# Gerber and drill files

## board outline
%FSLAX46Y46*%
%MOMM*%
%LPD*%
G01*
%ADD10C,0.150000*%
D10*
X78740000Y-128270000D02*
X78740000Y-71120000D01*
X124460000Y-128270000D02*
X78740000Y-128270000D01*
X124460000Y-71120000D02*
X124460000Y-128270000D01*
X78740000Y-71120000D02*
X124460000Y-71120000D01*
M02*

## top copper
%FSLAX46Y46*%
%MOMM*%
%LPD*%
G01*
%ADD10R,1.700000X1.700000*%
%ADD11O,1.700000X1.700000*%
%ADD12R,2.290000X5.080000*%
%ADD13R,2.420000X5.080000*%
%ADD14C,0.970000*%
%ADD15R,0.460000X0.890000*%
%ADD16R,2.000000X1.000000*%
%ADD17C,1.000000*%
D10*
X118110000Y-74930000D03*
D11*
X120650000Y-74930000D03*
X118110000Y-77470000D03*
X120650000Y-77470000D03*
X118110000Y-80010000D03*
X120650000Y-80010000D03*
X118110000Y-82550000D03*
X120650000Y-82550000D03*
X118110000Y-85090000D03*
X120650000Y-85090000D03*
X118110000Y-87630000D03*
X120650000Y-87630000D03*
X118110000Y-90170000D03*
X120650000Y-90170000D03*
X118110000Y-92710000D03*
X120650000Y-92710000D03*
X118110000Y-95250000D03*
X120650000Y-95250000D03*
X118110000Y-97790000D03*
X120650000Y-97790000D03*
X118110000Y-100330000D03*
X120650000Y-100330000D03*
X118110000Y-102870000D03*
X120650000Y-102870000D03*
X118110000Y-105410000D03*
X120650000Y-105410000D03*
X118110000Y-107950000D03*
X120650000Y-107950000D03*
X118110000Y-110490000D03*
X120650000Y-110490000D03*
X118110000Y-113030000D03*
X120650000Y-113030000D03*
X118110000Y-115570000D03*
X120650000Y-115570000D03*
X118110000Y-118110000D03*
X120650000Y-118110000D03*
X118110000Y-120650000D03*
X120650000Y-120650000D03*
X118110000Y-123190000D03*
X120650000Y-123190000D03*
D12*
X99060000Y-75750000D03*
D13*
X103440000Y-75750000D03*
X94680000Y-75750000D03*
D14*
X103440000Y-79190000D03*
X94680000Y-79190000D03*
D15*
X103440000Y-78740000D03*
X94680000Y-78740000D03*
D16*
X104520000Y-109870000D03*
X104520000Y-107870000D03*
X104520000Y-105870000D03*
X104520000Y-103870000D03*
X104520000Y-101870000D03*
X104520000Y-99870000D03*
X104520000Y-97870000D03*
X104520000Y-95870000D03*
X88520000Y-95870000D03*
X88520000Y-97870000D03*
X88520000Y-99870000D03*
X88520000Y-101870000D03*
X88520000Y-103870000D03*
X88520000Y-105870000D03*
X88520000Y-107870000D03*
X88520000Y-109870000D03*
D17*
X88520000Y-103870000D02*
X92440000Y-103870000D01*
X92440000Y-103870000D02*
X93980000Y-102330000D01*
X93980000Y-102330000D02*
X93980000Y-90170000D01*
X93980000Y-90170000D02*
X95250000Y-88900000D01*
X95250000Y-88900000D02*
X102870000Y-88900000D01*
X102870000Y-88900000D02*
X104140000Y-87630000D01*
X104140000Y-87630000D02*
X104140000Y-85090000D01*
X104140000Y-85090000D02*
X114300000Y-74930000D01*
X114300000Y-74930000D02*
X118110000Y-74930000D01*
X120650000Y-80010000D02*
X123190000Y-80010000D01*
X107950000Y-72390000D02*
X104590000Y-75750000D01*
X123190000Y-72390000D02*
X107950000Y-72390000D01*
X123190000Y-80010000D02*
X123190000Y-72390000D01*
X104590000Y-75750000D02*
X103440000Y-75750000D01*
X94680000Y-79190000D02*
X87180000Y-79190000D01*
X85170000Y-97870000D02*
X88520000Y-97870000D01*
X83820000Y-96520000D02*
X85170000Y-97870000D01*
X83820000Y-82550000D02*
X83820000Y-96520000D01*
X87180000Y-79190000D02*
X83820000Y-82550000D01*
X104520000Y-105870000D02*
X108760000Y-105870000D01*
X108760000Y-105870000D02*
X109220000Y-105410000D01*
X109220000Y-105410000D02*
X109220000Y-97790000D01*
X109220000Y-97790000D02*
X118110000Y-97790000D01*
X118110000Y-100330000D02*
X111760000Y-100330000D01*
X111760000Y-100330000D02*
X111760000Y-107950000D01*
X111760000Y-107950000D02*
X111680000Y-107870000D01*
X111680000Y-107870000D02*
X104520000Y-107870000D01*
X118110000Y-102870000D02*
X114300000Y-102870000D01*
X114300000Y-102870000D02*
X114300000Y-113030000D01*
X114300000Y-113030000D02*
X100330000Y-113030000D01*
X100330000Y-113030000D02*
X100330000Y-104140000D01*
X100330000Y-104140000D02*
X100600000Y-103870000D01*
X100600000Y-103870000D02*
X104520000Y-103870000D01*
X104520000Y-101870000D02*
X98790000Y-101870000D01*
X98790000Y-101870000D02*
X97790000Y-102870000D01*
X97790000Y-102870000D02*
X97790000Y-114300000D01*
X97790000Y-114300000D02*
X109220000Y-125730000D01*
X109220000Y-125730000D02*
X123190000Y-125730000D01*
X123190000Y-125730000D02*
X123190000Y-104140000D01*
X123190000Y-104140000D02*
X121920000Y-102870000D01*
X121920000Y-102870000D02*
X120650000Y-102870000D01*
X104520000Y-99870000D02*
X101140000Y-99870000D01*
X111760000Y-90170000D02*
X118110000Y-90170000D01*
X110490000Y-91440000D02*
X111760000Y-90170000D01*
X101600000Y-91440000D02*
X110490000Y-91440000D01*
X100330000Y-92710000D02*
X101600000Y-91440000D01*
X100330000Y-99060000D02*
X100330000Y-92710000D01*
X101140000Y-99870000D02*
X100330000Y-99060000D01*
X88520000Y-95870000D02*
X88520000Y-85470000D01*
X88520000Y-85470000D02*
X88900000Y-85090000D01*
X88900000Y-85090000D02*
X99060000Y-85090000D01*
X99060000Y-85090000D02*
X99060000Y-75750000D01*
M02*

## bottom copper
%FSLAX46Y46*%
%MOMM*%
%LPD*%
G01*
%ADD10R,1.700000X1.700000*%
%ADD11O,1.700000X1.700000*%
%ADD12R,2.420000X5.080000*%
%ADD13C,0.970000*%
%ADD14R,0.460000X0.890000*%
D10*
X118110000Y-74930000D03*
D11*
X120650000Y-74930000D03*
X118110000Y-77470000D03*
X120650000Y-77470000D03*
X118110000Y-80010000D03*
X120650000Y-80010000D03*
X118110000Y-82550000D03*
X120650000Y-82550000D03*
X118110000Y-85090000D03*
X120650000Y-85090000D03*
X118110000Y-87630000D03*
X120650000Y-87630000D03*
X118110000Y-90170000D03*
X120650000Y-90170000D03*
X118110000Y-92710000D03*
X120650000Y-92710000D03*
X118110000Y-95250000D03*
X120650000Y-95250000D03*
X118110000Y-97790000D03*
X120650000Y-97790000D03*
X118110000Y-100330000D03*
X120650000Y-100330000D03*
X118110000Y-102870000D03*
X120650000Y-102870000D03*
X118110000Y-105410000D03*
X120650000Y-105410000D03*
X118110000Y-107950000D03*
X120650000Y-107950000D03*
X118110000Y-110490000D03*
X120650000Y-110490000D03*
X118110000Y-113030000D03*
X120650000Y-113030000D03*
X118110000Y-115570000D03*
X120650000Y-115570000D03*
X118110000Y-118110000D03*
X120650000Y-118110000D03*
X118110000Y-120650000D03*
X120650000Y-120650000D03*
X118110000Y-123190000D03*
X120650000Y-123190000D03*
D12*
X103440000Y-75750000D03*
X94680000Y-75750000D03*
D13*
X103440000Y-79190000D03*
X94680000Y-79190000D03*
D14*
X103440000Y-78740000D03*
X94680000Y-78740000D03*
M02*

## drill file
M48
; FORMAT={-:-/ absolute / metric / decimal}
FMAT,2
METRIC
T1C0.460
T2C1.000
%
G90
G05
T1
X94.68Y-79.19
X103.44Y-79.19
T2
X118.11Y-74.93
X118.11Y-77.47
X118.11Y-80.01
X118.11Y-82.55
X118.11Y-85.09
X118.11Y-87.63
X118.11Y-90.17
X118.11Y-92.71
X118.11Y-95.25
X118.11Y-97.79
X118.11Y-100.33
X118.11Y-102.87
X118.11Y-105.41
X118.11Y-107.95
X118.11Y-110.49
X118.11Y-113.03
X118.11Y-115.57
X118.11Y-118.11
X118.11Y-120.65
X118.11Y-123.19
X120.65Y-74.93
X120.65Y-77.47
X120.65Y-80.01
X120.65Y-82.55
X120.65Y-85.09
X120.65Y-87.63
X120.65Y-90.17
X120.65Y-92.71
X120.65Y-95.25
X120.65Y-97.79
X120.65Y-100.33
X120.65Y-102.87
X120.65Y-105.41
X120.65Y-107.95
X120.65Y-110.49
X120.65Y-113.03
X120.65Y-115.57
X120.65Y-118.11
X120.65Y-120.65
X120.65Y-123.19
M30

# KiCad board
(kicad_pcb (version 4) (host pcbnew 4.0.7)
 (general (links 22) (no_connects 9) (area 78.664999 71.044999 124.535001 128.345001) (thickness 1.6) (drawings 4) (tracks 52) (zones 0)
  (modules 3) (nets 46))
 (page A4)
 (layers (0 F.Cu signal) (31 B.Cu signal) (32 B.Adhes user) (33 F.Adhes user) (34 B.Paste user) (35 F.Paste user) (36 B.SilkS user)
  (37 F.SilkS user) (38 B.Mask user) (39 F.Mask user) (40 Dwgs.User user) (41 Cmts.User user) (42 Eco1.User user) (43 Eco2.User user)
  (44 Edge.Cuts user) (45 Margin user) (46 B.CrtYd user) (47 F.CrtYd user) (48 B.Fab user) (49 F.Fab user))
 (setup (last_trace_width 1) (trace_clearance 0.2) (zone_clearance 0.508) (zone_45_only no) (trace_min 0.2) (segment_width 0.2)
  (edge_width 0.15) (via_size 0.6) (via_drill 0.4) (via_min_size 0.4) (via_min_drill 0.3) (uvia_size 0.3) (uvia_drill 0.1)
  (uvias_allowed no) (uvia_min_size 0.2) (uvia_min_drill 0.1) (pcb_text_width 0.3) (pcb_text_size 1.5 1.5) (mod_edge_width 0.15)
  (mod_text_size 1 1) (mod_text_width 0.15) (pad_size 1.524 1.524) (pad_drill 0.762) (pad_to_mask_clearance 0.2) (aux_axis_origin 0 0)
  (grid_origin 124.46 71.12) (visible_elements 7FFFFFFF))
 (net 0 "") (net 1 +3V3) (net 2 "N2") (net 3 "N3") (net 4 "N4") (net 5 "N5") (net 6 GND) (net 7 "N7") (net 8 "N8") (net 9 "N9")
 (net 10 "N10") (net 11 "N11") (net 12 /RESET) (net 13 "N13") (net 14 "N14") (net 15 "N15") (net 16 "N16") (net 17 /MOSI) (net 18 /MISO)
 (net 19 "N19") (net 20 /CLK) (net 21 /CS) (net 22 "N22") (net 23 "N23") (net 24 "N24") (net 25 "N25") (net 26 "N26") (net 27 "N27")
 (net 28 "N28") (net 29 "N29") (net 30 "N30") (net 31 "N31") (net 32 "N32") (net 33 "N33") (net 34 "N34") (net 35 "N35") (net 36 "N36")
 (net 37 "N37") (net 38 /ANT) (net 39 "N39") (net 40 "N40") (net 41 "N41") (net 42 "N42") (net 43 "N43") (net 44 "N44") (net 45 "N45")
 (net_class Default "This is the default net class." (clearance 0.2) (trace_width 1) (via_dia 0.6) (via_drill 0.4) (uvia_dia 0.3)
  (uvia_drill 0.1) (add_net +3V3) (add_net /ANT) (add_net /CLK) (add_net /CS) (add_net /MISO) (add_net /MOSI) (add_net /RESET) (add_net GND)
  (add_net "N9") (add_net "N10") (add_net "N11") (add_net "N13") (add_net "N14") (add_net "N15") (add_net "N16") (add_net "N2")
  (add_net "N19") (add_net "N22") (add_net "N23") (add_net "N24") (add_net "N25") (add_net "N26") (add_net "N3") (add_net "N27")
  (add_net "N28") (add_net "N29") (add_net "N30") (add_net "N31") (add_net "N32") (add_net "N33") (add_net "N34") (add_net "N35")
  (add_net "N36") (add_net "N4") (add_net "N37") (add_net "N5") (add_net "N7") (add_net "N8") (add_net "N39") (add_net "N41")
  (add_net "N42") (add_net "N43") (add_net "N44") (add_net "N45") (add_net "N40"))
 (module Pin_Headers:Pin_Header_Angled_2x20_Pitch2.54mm (layer F.Cu) (at 118.11 74.93)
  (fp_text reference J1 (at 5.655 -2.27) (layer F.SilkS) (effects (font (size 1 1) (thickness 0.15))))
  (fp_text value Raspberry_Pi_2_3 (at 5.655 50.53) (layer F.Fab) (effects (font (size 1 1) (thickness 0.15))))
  (pad 1 thru_hole rect (at 0 0) (size 1.7 1.7) (drill 1) (layers *.Cu *.Mask) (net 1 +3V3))
  (pad 2 thru_hole oval (at 2.54 0) (size 1.7 1.7) (drill 1) (layers *.Cu *.Mask) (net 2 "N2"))
  (pad 3 thru_hole oval (at 0 2.54) (size 1.7 1.7) (drill 1) (layers *.Cu *.Mask) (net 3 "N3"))
  (pad 4 thru_hole oval (at 2.54 2.54) (size 1.7 1.7) (drill 1) (layers *.Cu *.Mask) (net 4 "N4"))
  (pad 5 thru_hole oval (at 0 5.08) (size 1.7 1.7) (drill 1) (layers *.Cu *.Mask) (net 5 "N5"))
  (pad 6 thru_hole oval (at 2.54 5.08) (size 1.7 1.7) (drill 1) (layers *.Cu *.Mask) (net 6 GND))
  (pad 7 thru_hole oval (at 0 7.62) (size 1.7 1.7) (drill 1) (layers *.Cu *.Mask) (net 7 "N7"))
  (pad 8 thru_hole oval (at 2.54 7.62) (size 1.7 1.7) (drill 1) (layers *.Cu *.Mask) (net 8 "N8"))
  (pad 9 thru_hole oval (at 0 10.16) (size 1.7 1.7) (drill 1) (layers *.Cu *.Mask) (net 6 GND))
  (pad 10 thru_hole oval (at 2.54 10.16) (size 1.7 1.7) (drill 1) (layers *.Cu *.Mask) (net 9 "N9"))
  (pad 11 thru_hole oval (at 0 12.7) (size 1.7 1.7) (drill 1) (layers *.Cu *.Mask) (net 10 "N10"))
  (pad 12 thru_hole oval (at 2.54 12.7) (size 1.7 1.7) (drill 1) (layers *.Cu *.Mask) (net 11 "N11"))
  (pad 13 thru_hole oval (at 0 15.24) (size 1.7 1.7) (drill 1) (layers *.Cu *.Mask) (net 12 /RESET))
  (pad 14 thru_hole oval (at 2.54 15.24) (size 1.7 1.7) (drill 1) (layers *.Cu *.Mask) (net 6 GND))
  (pad 15 thru_hole oval (at 0 17.78) (size 1.7 1.7) (drill 1) (layers *.Cu *.Mask) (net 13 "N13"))
  (pad 16 thru_hole oval (at 2.54 17.78) (size 1.7 1.7) (drill 1) (layers *.Cu *.Mask) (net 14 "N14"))
  (pad 17 thru_hole oval (at 0 20.32) (size 1.7 1.7) (drill 1) (layers *.Cu *.Mask) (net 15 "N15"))
  (pad 18 thru_hole oval (at 2.54 20.32) (size 1.7 1.7) (drill 1) (layers *.Cu *.Mask) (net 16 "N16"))
  (pad 19 thru_hole oval (at 0 22.86) (size 1.7 1.7) (drill 1) (layers *.Cu *.Mask) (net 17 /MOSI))
  (pad 20 thru_hole oval (at 2.54 22.86) (size 1.7 1.7) (drill 1) (layers *.Cu *.Mask) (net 6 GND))
  (pad 21 thru_hole oval (at 0 25.4) (size 1.7 1.7) (drill 1) (layers *.Cu *.Mask) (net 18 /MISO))
  (pad 22 thru_hole oval (at 2.54 25.4) (size 1.7 1.7) (drill 1) (layers *.Cu *.Mask) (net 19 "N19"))
  (pad 23 thru_hole oval (at 0 27.94) (size 1.7 1.7) (drill 1) (layers *.Cu *.Mask) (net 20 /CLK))
  (pad 24 thru_hole oval (at 2.54 27.94) (size 1.7 1.7) (drill 1) (layers *.Cu *.Mask) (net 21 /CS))
  (pad 25 thru_hole oval (at 0 30.48) (size 1.7 1.7) (drill 1) (layers *.Cu *.Mask) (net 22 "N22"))
  (pad 26 thru_hole oval (at 2.54 30.48) (size 1.7 1.7) (drill 1) (layers *.Cu *.Mask) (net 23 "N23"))
  (pad 27 thru_hole oval (at 0 33.02) (size 1.7 1.7) (drill 1) (layers *.Cu *.Mask) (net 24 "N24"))
  (pad 28 thru_hole oval (at 2.54 33.02) (size 1.7 1.7) (drill 1) (layers *.Cu *.Mask) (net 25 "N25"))
  (pad 29 thru_hole oval (at 0 35.56) (size 1.7 1.7) (drill 1) (layers *.Cu *.Mask) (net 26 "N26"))
  (pad 30 thru_hole oval (at 2.54 35.56) (size 1.7 1.7) (drill 1) (layers *.Cu *.Mask) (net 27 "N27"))
  (pad 31 thru_hole oval (at 0 38.1) (size 1.7 1.7) (drill 1) (layers *.Cu *.Mask) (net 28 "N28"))
  (pad 32 thru_hole oval (at 2.54 38.1) (size 1.7 1.7) (drill 1) (layers *.Cu *.Mask) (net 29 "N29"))
  (pad 33 thru_hole oval (at 0 40.64) (size 1.7 1.7) (drill 1) (layers *.Cu *.Mask) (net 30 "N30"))
  (pad 34 thru_hole oval (at 2.54 40.64) (size 1.7 1.7) (drill 1) (layers *.Cu *.Mask) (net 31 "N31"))
  (pad 35 thru_hole oval (at 0 43.18) (size 1.7 1.7) (drill 1) (layers *.Cu *.Mask) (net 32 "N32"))
  (pad 36 thru_hole oval (at 2.54 43.18) (size 1.7 1.7) (drill 1) (layers *.Cu *.Mask) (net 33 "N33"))
  (pad 37 thru_hole oval (at 0 45.72) (size 1.7 1.7) (drill 1) (layers *.Cu *.Mask) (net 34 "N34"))
  (pad 38 thru_hole oval (at 2.54 45.72) (size 1.7 1.7) (drill 1) (layers *.Cu *.Mask) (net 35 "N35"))
  (pad 39 thru_hole oval (at 0 48.26) (size 1.7 1.7) (drill 1) (layers *.Cu *.Mask) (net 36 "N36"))
  (pad 40 thru_hole oval (at 2.54 48.26) (size 1.7 1.7) (drill 1) (layers *.Cu *.Mask) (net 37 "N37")))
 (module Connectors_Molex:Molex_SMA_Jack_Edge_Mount (layer F.Cu) (at 99.06 77.47 270)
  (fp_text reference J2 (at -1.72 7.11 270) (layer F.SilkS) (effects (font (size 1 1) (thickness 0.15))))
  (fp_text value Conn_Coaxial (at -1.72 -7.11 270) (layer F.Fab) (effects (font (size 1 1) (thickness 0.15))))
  (pad 1 smd rect (at -1.72 0 270) (size 5.08 2.29) (layers F.Cu F.Paste F.Mask) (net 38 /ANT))
  (pad 2 smd rect (at -1.72 -4.38 270) (size 5.08 2.42) (layers F.Cu F.Paste F.Mask) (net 6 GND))
  (pad 2 smd rect (at -1.72 4.38 270) (size 5.08 2.42) (layers F.Cu F.Paste F.Mask) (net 6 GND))
  (pad 2 smd rect (at -1.72 -4.38 270) (size 5.08 2.42) (layers B.Cu B.Paste B.Mask) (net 6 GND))
  (pad 2 smd rect (at -1.72 4.38 270) (size 5.08 2.42) (layers B.Cu B.Paste B.Mask) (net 6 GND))
  (pad 2 thru_hole circle (at 1.72 -4.38 270) (size 0.97 0.97) (drill 0.46) (layers *.Cu) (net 6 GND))
  (pad 2 thru_hole circle (at 1.72 4.38 270) (size 0.97 0.97) (drill 0.46) (layers *.Cu) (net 6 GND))
  (pad 2 smd rect (at 1.27 -4.38 270) (size 0.89 0.46) (layers F.Cu) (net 6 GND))
  (pad 2 smd rect (at 1.27 4.38 270) (size 0.89 0.46) (layers F.Cu) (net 6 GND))
  (pad 2 smd rect (at 1.27 -4.38 270) (size 0.89 0.46) (layers B.Cu) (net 6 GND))
  (pad 2 smd rect (at 1.27 4.38 270) (size 0.89 0.46) (layers B.Cu) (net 6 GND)))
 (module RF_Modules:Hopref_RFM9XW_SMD (layer F.Cu) (at 96.52 102.87 180)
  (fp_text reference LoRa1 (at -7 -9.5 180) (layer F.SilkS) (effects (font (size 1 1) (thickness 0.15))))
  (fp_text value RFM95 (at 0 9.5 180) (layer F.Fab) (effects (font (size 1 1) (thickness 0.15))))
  (pad 1 smd rect (at -8 -7 180) (size 2 1) (layers F.Cu F.Paste F.Mask) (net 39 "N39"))
  (pad 2 smd rect (at -8 -5 180) (size 2 1) (layers F.Cu F.Paste F.Mask) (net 18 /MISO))
  (pad 3 smd rect (at -8 -3 180) (size 2 1) (layers F.Cu F.Paste F.Mask) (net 17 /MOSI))
  (pad 4 smd rect (at -8 -1 180) (size 2 1) (layers F.Cu F.Paste F.Mask) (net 20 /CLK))
  (pad 5 smd rect (at -8 1 180) (size 2 1) (layers F.Cu F.Paste F.Mask) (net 21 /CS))
  (pad 6 smd rect (at -8 3 180) (size 2 1) (layers F.Cu F.Paste F.Mask) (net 12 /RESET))
  (pad 7 smd rect (at -8 5 180) (size 2 1) (layers F.Cu F.Paste F.Mask) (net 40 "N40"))
  (pad 8 smd rect (at -8 7 180) (size 2 1) (layers F.Cu F.Paste F.Mask) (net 6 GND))
  (pad 9 smd rect (at 8 7 180) (size 2 1) (layers F.Cu F.Paste F.Mask) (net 38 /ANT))
  (pad 10 smd rect (at 8 5 180) (size 2 1) (layers F.Cu F.Paste F.Mask) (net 6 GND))
  (pad 11 smd rect (at 8 3 180) (size 2 1) (layers F.Cu F.Paste F.Mask) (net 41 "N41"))
  (pad 12 smd rect (at 8 1 180) (size 2 1) (layers F.Cu F.Paste F.Mask) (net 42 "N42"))
  (pad 13 smd rect (at 8 -1 180) (size 2 1) (layers F.Cu F.Paste F.Mask) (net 1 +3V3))
  (pad 14 smd rect (at 8 -3 180) (size 2 1) (layers F.Cu F.Paste F.Mask) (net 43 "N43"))
  (pad 15 smd rect (at 8 -5 180) (size 2 1) (layers F.Cu F.Paste F.Mask) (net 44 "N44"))
  (pad 16 smd rect (at 8 -7 180) (size 2 1) (layers F.Cu F.Paste F.Mask) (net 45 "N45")))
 (gr_line (start 78.74 128.27) (end 78.74 71.12) (angle 90) (layer Edge.Cuts) (width 0.15))
 (gr_line (start 124.46 128.27) (end 78.74 128.27) (angle 90) (layer Edge.Cuts) (width 0.15))
 (gr_line (start 124.46 71.12) (end 124.46 128.27) (angle 90) (layer Edge.Cuts) (width 0.15))
 (gr_line (start 78.74 71.12) (end 124.46 71.12) (angle 90) (layer Edge.Cuts) (width 0.15))
 (segment (start 88.52 103.87) (end 92.44 103.87) (width 1) (layer F.Cu) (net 1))
 (segment (start 92.44 103.87) (end 93.98 102.33) (width 1) (layer F.Cu) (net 1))
 (segment (start 93.98 102.33) (end 93.98 90.17) (width 1) (layer F.Cu) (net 1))
 (segment (start 93.98 90.17) (end 95.25 88.9) (width 1) (layer F.Cu) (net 1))
 (segment (start 95.25 88.9) (end 102.87 88.9) (width 1) (layer F.Cu) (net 1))
 (segment (start 102.87 88.9) (end 104.14 87.63) (width 1) (layer F.Cu) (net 1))
 (segment (start 104.14 87.63) (end 104.14 85.09) (width 1) (layer F.Cu) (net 1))
 (segment (start 104.14 85.09) (end 114.3 74.93) (width 1) (layer F.Cu) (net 1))
 (segment (start 114.3 74.93) (end 118.11 74.93) (width 1) (layer F.Cu) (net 1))
 (segment (start 120.65 80.01) (end 123.19 80.01) (width 1) (layer F.Cu) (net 6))
 (segment (start 107.95 72.39) (end 104.59 75.75) (width 1) (layer F.Cu) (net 6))
 (segment (start 123.19 72.39) (end 107.95 72.39) (width 1) (layer F.Cu) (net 6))
 (segment (start 123.19 80.01) (end 123.19 72.39) (width 1) (layer F.Cu) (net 6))
 (segment (start 104.59 75.75) (end 103.44 75.75) (width 1) (layer F.Cu) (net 6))
 (segment (start 94.68 79.19) (end 87.18 79.19) (width 1) (layer F.Cu) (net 6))
 (segment (start 85.17 97.87) (end 88.52 97.87) (width 1) (layer F.Cu) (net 6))
 (segment (start 83.82 96.52) (end 85.17 97.87) (width 1) (layer F.Cu) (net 6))
 (segment (start 83.82 82.55) (end 83.82 96.52) (width 1) (layer F.Cu) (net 6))
 (segment (start 87.18 79.19) (end 83.82 82.55) (width 1) (layer F.Cu) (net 6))
 (segment (start 104.52 105.87) (end 108.76 105.87) (width 1) (layer F.Cu) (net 17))
 (segment (start 108.76 105.87) (end 109.22 105.41) (width 1) (layer F.Cu) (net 17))
 (segment (start 109.22 105.41) (end 109.22 97.79) (width 1) (layer F.Cu) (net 17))
 (segment (start 109.22 97.79) (end 118.11 97.79) (width 1) (layer F.Cu) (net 17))
 (segment (start 118.11 100.33) (end 111.76 100.33) (width 1) (layer F.Cu) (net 18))
 (segment (start 111.76 100.33) (end 111.76 107.95) (width 1) (layer F.Cu) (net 18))
 (segment (start 111.76 107.95) (end 111.68 107.87) (width 1) (layer F.Cu) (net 18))
 (segment (start 111.68 107.87) (end 104.52 107.87) (width 1) (layer F.Cu) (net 18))
 (segment (start 118.11 102.87) (end 114.3 102.87) (width 1) (layer F.Cu) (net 20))
 (segment (start 114.3 102.87) (end 114.3 113.03) (width 1) (layer F.Cu) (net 20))
 (segment (start 114.3 113.03) (end 100.33 113.03) (width 1) (layer F.Cu) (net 20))
 (segment (start 100.33 113.03) (end 100.33 104.14) (width 1) (layer F.Cu) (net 20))
 (segment (start 100.33 104.14) (end 100.6 103.87) (width 1) (layer F.Cu) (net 20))
 (segment (start 100.6 103.87) (end 104.52 103.87) (width 1) (layer F.Cu) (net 20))
 (segment (start 104.52 101.87) (end 98.79 101.87) (width 1) (layer F.Cu) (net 21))
 (segment (start 98.79 101.87) (end 97.79 102.87) (width 1) (layer F.Cu) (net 21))
 (segment (start 97.79 102.87) (end 97.79 114.3) (width 1) (layer F.Cu) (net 21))
 (segment (start 97.79 114.3) (end 109.22 125.73) (width 1) (layer F.Cu) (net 21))
 (segment (start 109.22 125.73) (end 123.19 125.73) (width 1) (layer F.Cu) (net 21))
 (segment (start 123.19 125.73) (end 123.19 104.14) (width 1) (layer F.Cu) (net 21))
 (segment (start 123.19 104.14) (end 121.92 102.87) (width 1) (layer F.Cu) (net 21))
 (segment (start 121.92 102.87) (end 120.65 102.87) (width 1) (layer F.Cu) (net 21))
 (segment (start 104.52 99.87) (end 101.14 99.87) (width 1) (layer F.Cu) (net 12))
 (segment (start 111.76 90.17) (end 118.11 90.17) (width 1) (layer F.Cu) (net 12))
 (segment (start 110.49 91.44) (end 111.76 90.17) (width 1) (layer F.Cu) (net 12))
 (segment (start 101.6 91.44) (end 110.49 91.44) (width 1) (layer F.Cu) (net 12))
 (segment (start 100.33 92.71) (end 101.6 91.44) (width 1) (layer F.Cu) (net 12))
 (segment (start 100.33 99.06) (end 100.33 92.71) (width 1) (layer F.Cu) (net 12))
 (segment (start 101.14 99.87) (end 100.33 99.06) (width 1) (layer F.Cu) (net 12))
 (segment (start 88.52 95.87) (end 88.52 85.47) (width 1) (layer F.Cu) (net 38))
 (segment (start 88.52 85.47) (end 88.9 85.09) (width 1) (layer F.Cu) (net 38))
 (segment (start 88.9 85.09) (end 99.06 85.09) (width 1) (layer F.Cu) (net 38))
 (segment (start 99.06 85.09) (end 99.06 75.75) (width 1) (layer F.Cu) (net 38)))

